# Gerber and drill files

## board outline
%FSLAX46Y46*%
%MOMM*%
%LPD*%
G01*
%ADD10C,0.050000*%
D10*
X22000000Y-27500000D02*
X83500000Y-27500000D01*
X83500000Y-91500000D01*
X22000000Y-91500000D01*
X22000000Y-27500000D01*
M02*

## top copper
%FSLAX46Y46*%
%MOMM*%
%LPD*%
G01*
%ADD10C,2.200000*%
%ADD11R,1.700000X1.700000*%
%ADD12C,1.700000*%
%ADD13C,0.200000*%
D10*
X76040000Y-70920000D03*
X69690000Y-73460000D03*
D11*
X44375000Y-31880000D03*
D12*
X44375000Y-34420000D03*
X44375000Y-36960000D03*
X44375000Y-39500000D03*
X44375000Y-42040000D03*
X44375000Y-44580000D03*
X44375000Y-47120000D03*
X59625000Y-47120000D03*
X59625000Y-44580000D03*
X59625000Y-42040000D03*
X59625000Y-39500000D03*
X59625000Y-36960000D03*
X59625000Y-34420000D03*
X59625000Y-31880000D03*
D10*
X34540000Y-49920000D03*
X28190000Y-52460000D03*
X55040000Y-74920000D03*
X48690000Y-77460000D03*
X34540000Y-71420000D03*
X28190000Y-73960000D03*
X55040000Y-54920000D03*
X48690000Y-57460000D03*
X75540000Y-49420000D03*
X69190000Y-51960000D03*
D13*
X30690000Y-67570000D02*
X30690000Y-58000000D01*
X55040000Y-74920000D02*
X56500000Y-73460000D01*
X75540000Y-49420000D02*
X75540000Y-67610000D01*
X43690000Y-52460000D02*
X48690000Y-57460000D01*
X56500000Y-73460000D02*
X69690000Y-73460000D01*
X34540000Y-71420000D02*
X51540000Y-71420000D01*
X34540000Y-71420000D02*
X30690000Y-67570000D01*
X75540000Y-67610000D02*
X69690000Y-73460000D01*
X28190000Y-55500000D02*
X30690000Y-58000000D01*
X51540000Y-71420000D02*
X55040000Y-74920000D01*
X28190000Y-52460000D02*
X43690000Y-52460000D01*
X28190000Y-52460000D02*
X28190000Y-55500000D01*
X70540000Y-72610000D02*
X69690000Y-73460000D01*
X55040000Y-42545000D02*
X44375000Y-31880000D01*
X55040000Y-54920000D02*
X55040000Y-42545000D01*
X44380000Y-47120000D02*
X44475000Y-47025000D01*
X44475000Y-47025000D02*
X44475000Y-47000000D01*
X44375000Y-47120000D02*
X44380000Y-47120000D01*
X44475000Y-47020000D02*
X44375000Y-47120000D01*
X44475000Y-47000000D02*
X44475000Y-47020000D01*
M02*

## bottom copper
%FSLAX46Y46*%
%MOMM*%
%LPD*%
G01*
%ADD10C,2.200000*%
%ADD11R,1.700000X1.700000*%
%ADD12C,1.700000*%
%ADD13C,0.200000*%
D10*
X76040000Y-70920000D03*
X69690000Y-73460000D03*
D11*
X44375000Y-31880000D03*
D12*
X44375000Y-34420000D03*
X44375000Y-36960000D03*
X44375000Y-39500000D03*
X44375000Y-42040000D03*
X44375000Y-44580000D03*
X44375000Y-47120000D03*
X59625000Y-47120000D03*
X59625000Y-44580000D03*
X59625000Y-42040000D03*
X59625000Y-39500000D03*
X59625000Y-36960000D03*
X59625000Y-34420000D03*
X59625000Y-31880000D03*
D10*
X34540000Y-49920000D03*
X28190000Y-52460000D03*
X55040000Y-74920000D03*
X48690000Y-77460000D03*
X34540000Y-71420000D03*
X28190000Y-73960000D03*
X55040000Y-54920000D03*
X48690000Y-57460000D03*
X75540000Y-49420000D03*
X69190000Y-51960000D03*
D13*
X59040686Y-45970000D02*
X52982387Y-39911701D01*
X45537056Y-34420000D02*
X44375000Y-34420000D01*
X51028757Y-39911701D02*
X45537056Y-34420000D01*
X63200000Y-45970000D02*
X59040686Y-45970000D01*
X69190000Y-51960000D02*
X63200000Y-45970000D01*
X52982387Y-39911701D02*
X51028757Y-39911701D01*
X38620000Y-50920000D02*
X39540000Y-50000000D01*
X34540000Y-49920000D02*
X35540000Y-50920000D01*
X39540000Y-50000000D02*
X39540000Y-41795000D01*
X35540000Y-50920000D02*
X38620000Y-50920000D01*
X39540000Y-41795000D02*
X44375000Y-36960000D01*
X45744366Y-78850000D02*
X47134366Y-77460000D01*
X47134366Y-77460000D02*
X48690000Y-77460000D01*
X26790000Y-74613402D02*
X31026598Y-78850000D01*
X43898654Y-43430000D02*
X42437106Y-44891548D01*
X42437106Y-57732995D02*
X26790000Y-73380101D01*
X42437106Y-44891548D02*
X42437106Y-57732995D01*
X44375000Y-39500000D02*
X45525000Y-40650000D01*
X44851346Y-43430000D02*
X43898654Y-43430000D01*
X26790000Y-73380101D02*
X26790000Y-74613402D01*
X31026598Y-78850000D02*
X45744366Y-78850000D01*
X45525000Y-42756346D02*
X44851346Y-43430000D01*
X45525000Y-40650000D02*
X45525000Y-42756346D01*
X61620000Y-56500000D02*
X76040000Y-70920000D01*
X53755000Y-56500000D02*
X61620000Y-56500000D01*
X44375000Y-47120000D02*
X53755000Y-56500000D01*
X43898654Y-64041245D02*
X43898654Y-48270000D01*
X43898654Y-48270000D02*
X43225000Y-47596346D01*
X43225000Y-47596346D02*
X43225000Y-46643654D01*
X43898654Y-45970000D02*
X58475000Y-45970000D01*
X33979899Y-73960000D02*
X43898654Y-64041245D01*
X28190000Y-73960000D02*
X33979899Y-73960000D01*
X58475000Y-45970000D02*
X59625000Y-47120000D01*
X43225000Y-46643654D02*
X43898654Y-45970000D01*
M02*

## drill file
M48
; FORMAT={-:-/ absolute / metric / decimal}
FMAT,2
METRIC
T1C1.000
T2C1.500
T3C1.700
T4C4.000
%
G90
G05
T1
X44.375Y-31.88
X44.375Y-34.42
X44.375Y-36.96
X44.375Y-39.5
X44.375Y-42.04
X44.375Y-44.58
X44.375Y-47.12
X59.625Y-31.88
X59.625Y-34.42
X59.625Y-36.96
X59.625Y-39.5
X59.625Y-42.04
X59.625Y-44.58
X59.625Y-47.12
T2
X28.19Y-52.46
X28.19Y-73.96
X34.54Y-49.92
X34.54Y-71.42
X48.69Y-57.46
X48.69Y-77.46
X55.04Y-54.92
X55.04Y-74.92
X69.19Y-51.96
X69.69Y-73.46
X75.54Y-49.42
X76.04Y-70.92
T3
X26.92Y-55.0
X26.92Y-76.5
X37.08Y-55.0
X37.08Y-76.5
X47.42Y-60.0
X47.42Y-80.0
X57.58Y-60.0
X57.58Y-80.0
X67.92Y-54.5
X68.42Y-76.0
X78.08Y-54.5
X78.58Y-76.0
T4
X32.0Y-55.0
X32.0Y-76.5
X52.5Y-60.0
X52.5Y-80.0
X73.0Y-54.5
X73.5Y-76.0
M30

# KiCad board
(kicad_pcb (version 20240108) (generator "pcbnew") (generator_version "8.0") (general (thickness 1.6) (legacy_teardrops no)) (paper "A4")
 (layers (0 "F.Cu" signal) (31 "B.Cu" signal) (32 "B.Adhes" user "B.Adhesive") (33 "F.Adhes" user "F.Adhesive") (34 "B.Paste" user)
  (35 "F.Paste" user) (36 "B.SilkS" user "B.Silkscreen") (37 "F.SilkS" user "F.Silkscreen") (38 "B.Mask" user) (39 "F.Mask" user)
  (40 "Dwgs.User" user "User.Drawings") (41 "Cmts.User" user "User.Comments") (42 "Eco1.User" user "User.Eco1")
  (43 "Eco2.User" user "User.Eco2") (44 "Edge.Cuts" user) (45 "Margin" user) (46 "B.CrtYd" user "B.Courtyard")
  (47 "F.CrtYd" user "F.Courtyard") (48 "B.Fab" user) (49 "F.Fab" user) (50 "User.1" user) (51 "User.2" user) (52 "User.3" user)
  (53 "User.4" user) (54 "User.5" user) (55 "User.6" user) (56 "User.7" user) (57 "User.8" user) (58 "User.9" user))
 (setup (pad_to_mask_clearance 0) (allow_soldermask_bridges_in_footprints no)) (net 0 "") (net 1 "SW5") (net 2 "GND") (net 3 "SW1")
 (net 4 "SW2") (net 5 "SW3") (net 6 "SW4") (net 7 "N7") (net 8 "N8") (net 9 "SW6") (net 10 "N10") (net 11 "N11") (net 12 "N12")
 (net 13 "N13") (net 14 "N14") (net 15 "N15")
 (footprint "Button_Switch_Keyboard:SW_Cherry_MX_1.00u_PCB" (layer "F.Cu") (at 76.04 70.92)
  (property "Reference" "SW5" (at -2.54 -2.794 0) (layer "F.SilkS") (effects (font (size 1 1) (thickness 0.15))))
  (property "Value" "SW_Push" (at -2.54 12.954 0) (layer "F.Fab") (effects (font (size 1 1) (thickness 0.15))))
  (pad "" np_thru_hole circle (at -7.62 5.08) (size 1.7 1.7) (drill 1.7) (layers "*.Cu" "*.Mask"))
  (pad "" np_thru_hole circle (at -2.54 5.08) (size 4 4) (drill 4) (layers "*.Cu" "*.Mask"))
  (pad "" np_thru_hole circle (at 2.54 5.08) (size 1.7 1.7) (drill 1.7) (layers "*.Cu" "*.Mask"))
  (pad "1" thru_hole circle (at 0 0) (size 2.2 2.2) (drill 1.5) (layers "*.Cu" "*.Mask") (remove_unused_layers no) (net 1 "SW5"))
  (pad "2" thru_hole circle (at -6.35 2.54) (size 2.2 2.2) (drill 1.5) (layers "*.Cu" "*.Mask") (remove_unused_layers no) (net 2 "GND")))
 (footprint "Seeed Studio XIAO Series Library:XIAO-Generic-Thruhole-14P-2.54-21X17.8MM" (layer "F.Cu") (at 52 39.5)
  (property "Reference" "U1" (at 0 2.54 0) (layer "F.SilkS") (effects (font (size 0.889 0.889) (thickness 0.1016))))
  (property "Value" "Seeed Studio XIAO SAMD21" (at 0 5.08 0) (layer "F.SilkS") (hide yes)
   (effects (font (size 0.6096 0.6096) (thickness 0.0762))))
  (pad "1" thru_hole rect (at -7.625 -7.62) (size 1.7 1.7) (drill 1) (layers "*.Cu" "*.Mask") (remove_unused_layers no) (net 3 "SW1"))
  (pad "2" thru_hole circle (at -7.625 -5.08) (size 1.7 1.7) (drill 1) (layers "*.Cu" "*.Mask") (remove_unused_layers no) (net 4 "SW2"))
  (pad "3" thru_hole circle (at -7.625 -2.54) (size 1.7 1.7) (drill 1) (layers "*.Cu" "*.Mask") (remove_unused_layers no) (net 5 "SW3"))
  (pad "4" thru_hole circle (at -7.625 0) (size 1.7 1.7) (drill 1) (layers "*.Cu" "*.Mask") (remove_unused_layers no) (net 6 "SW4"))
  (pad "5" thru_hole circle (at -7.625 2.54) (size 1.7 1.7) (drill 1) (layers "*.Cu" "*.Mask") (remove_unused_layers no) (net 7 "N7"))
  (pad "6" thru_hole circle (at -7.625 5.08 180) (size 1.7 1.7) (drill 1) (layers "*.Cu" "*.Mask") (remove_unused_layers no) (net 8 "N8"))
  (pad "7" thru_hole circle (at -7.625 7.62) (size 1.7 1.7) (drill 1) (layers "*.Cu" "*.Mask") (remove_unused_layers no) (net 1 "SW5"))
  (pad "8" thru_hole circle (at 7.625 7.62) (size 1.7 1.7) (drill 1) (layers "*.Cu" "*.Mask") (remove_unused_layers no) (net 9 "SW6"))
  (pad "9" thru_hole circle (at 7.625 5.08) (size 1.7 1.7) (drill 1) (layers "*.Cu" "*.Mask") (remove_unused_layers no) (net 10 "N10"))
  (pad "10" thru_hole circle (at 7.625 2.54) (size 1.7 1.7) (drill 1) (layers "*.Cu" "*.Mask") (remove_unused_layers no) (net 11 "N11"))
  (pad "11" thru_hole circle (at 7.625 0) (size 1.7 1.7) (drill 1) (layers "*.Cu" "*.Mask") (remove_unused_layers no) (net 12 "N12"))
  (pad "12" thru_hole circle (at 7.625 -2.54) (size 1.7 1.7) (drill 1) (layers "*.Cu" "*.Mask") (remove_unused_layers no) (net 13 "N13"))
  (pad "13" thru_hole circle (at 7.625 -5.08) (size 1.7 1.7) (drill 1) (layers "*.Cu" "*.Mask") (remove_unused_layers no) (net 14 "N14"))
  (pad "14" thru_hole circle (at 7.625 -7.62) (size 1.7 1.7) (drill 1) (layers "*.Cu" "*.Mask") (remove_unused_layers no) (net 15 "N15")))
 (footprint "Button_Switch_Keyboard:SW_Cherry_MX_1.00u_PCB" (layer "F.Cu") (at 34.54 49.92)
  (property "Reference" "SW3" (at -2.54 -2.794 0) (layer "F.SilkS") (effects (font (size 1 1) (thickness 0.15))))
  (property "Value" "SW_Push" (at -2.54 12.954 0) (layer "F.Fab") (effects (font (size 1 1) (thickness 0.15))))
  (pad "" np_thru_hole circle (at -7.62 5.08) (size 1.7 1.7) (drill 1.7) (layers "*.Cu" "*.Mask"))
  (pad "" np_thru_hole circle (at -2.54 5.08) (size 4 4) (drill 4) (layers "*.Cu" "*.Mask"))
  (pad "" np_thru_hole circle (at 2.54 5.08) (size 1.7 1.7) (drill 1.7) (layers "*.Cu" "*.Mask"))
  (pad "1" thru_hole circle (at 0 0) (size 2.2 2.2) (drill 1.5) (layers "*.Cu" "*.Mask") (remove_unused_layers no) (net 5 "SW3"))
  (pad "2" thru_hole circle (at -6.35 2.54) (size 2.2 2.2) (drill 1.5) (layers "*.Cu" "*.Mask") (remove_unused_layers no) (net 2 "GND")))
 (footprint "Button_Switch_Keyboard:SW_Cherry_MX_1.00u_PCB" (layer "F.Cu") (at 55.04 74.92)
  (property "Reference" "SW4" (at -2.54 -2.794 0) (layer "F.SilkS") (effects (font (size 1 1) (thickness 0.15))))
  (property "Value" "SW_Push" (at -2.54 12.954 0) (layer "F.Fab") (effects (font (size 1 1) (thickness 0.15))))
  (pad "" np_thru_hole circle (at -7.62 5.08) (size 1.7 1.7) (drill 1.7) (layers "*.Cu" "*.Mask"))
  (pad "" np_thru_hole circle (at -2.54 5.08) (size 4 4) (drill 4) (layers "*.Cu" "*.Mask"))
  (pad "" np_thru_hole circle (at 2.54 5.08) (size 1.7 1.7) (drill 1.7) (layers "*.Cu" "*.Mask"))
  (pad "1" thru_hole circle (at 0 0) (size 2.2 2.2) (drill 1.5) (layers "*.Cu" "*.Mask") (remove_unused_layers no) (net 2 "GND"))
  (pad "2" thru_hole circle (at -6.35 2.54) (size 2.2 2.2) (drill 1.5) (layers "*.Cu" "*.Mask") (remove_unused_layers no) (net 6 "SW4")))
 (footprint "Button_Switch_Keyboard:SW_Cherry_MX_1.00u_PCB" (layer "F.Cu") (at 34.54 71.42)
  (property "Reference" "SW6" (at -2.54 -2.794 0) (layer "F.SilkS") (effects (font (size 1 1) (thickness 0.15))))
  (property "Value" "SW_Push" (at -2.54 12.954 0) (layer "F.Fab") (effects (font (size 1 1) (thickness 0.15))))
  (pad "" np_thru_hole circle (at -7.62 5.08) (size 1.7 1.7) (drill 1.7) (layers "*.Cu" "*.Mask"))
  (pad "" np_thru_hole circle (at -2.54 5.08) (size 4 4) (drill 4) (layers "*.Cu" "*.Mask"))
  (pad "" np_thru_hole circle (at 2.54 5.08) (size 1.7 1.7) (drill 1.7) (layers "*.Cu" "*.Mask"))
  (pad "1" thru_hole circle (at 0 0) (size 2.2 2.2) (drill 1.5) (layers "*.Cu" "*.Mask") (remove_unused_layers no) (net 2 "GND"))
  (pad "2" thru_hole circle (at -6.35 2.54) (size 2.2 2.2) (drill 1.5) (layers "*.Cu" "*.Mask") (remove_unused_layers no) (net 9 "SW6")))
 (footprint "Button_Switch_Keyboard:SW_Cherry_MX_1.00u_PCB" (layer "F.Cu") (at 55.04 54.92)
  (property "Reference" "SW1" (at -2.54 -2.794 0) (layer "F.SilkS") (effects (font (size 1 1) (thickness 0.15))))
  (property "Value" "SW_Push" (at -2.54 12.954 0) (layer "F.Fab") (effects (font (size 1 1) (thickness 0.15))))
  (pad "" np_thru_hole circle (at -7.62 5.08) (size 1.7 1.7) (drill 1.7) (layers "*.Cu" "*.Mask"))
  (pad "" np_thru_hole circle (at -2.54 5.08) (size 4 4) (drill 4) (layers "*.Cu" "*.Mask"))
  (pad "" np_thru_hole circle (at 2.54 5.08) (size 1.7 1.7) (drill 1.7) (layers "*.Cu" "*.Mask"))
  (pad "1" thru_hole circle (at 0 0) (size 2.2 2.2) (drill 1.5) (layers "*.Cu" "*.Mask") (remove_unused_layers no) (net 3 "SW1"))
  (pad "2" thru_hole circle (at -6.35 2.54) (size 2.2 2.2) (drill 1.5) (layers "*.Cu" "*.Mask") (remove_unused_layers no) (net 2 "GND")))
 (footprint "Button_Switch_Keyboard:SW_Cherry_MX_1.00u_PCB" (layer "F.Cu") (at 75.54 49.42)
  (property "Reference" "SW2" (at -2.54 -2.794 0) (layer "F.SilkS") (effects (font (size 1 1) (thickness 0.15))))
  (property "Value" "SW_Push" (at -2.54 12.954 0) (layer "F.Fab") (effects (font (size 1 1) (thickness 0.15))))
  (pad "" np_thru_hole circle (at -7.62 5.08) (size 1.7 1.7) (drill 1.7) (layers "*.Cu" "*.Mask"))
  (pad "" np_thru_hole circle (at -2.54 5.08) (size 4 4) (drill 4) (layers "*.Cu" "*.Mask"))
  (pad "" np_thru_hole circle (at 2.54 5.08) (size 1.7 1.7) (drill 1.7) (layers "*.Cu" "*.Mask"))
  (pad "1" thru_hole circle (at 0 0) (size 2.2 2.2) (drill 1.5) (layers "*.Cu" "*.Mask") (remove_unused_layers no) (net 2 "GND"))
  (pad "2" thru_hole circle (at -6.35 2.54) (size 2.2 2.2) (drill 1.5) (layers "*.Cu" "*.Mask") (remove_unused_layers no) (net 4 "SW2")))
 (gr_rect (start 22 27.5) (end 83.5 91.5) (stroke (width 0.05) (type default)) (fill none) (layer "Edge.Cuts"))
 (segment (start 30.69 67.57) (end 30.69 58) (width 0.2) (layer "F.Cu") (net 2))
 (segment (start 55.04 74.92) (end 56.5 73.46) (width 0.2) (layer "F.Cu") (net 2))
 (segment (start 75.54 49.42) (end 75.54 67.61) (width 0.2) (layer "F.Cu") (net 2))
 (segment (start 43.69 52.46) (end 48.69 57.46) (width 0.2) (layer "F.Cu") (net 2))
 (segment (start 56.5 73.46) (end 69.69 73.46) (width 0.2) (layer "F.Cu") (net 2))
 (segment (start 34.54 71.42) (end 51.54 71.42) (width 0.2) (layer "F.Cu") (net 2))
 (segment (start 34.54 71.42) (end 30.69 67.57) (width 0.2) (layer "F.Cu") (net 2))
 (segment (start 75.54 67.61) (end 69.69 73.46) (width 0.2) (layer "F.Cu") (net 2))
 (segment (start 28.19 55.5) (end 30.69 58) (width 0.2) (layer "F.Cu") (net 2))
 (segment (start 51.54 71.42) (end 55.04 74.92) (width 0.2) (layer "F.Cu") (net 2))
 (segment (start 28.19 52.46) (end 43.69 52.46) (width 0.2) (layer "F.Cu") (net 2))
 (segment (start 28.19 52.46) (end 28.19 55.5) (width 0.2) (layer "F.Cu") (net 2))
 (segment (start 70.54 72.61) (end 69.69 73.46) (width 0.2) (layer "F.Cu") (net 2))
 (segment (start 55.04 42.545) (end 44.375 31.88) (width 0.2) (layer "F.Cu") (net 3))
 (segment (start 55.04 54.92) (end 55.04 42.545) (width 0.2) (layer "F.Cu") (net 3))
 (segment (start 59.040686 45.97) (end 52.982387 39.911701) (width 0.2) (layer "B.Cu") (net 4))
 (segment (start 45.537056 34.42) (end 44.375 34.42) (width 0.2) (layer "B.Cu") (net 4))
 (segment (start 51.028757 39.911701) (end 45.537056 34.42) (width 0.2) (layer "B.Cu") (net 4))
 (segment (start 63.2 45.97) (end 59.040686 45.97) (width 0.2) (layer "B.Cu") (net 4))
 (segment (start 69.19 51.96) (end 63.2 45.97) (width 0.2) (layer "B.Cu") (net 4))
 (segment (start 52.982387 39.911701) (end 51.028757 39.911701) (width 0.2) (layer "B.Cu") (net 4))
 (segment (start 38.62 50.92) (end 39.54 50) (width 0.2) (layer "B.Cu") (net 5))
 (segment (start 34.54 49.92) (end 35.54 50.92) (width 0.2) (layer "B.Cu") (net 5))
 (segment (start 39.54 50) (end 39.54 41.795) (width 0.2) (layer "B.Cu") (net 5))
 (segment (start 35.54 50.92) (end 38.62 50.92) (width 0.2) (layer "B.Cu") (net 5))
 (segment (start 39.54 41.795) (end 44.375 36.96) (width 0.2) (layer "B.Cu") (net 5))
 (segment (start 45.744366 78.85) (end 47.134366 77.46) (width 0.2) (layer "B.Cu") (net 6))
 (segment (start 47.134366 77.46) (end 48.69 77.46) (width 0.2) (layer "B.Cu") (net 6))
 (segment (start 26.79 74.613402) (end 31.026598 78.85) (width 0.2) (layer "B.Cu") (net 6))
 (segment (start 43.898654 43.43) (end 42.437106 44.891548) (width 0.2) (layer "B.Cu") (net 6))
 (segment (start 42.437106 57.732995) (end 26.79 73.380101) (width 0.2) (layer "B.Cu") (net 6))
 (segment (start 42.437106 44.891548) (end 42.437106 57.732995) (width 0.2) (layer "B.Cu") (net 6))
 (segment (start 44.375 39.5) (end 45.525 40.65) (width 0.2) (layer "B.Cu") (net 6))
 (segment (start 44.851346 43.43) (end 43.898654 43.43) (width 0.2) (layer "B.Cu") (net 6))
 (segment (start 26.79 73.380101) (end 26.79 74.613402) (width 0.2) (layer "B.Cu") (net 6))
 (segment (start 31.026598 78.85) (end 45.744366 78.85) (width 0.2) (layer "B.Cu") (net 6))
 (segment (start 45.525 42.756346) (end 44.851346 43.43) (width 0.2) (layer "B.Cu") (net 6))
 (segment (start 45.525 40.65) (end 45.525 42.756346) (width 0.2) (layer "B.Cu") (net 6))
 (segment (start 44.38 47.12) (end 44.475 47.025) (width 0.2) (layer "F.Cu") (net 1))
 (segment (start 44.475 47.025) (end 44.475 47) (width 0.2) (layer "F.Cu") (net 1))
 (segment (start 44.375 47.12) (end 44.38 47.12) (width 0.2) (layer "F.Cu") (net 1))
 (segment (start 44.475 47.02) (end 44.375 47.12) (width 0.2) (layer "F.Cu") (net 1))
 (segment (start 44.475 47) (end 44.475 47.02) (width 0.2) (layer "F.Cu") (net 1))
 (segment (start 61.62 56.5) (end 76.04 70.92) (width 0.2) (layer "B.Cu") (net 1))
 (segment (start 53.755 56.5) (end 61.62 56.5) (width 0.2) (layer "B.Cu") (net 1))
 (segment (start 44.375 47.12) (end 53.755 56.5) (width 0.2) (layer "B.Cu") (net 1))
 (segment (start 43.898654 64.041245) (end 43.898654 48.27) (width 0.2) (layer "B.Cu") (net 9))
 (segment (start 43.898654 48.27) (end 43.225 47.596346) (width 0.2) (layer "B.Cu") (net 9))
 (segment (start 43.225 47.596346) (end 43.225 46.643654) (width 0.2) (layer "B.Cu") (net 9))
 (segment (start 43.898654 45.97) (end 58.475 45.97) (width 0.2) (layer "B.Cu") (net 9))
 (segment (start 33.979899 73.96) (end 43.898654 64.041245) (width 0.2) (layer "B.Cu") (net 9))
 (segment (start 28.19 73.96) (end 33.979899 73.96) (width 0.2) (layer "B.Cu") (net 9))
 (segment (start 58.475 45.97) (end 59.625 47.12) (width 0.2) (layer "B.Cu") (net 9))
 (segment (start 43.225 46.643654) (end 43.898654 45.97) (width 0.2) (layer "B.Cu") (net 9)))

